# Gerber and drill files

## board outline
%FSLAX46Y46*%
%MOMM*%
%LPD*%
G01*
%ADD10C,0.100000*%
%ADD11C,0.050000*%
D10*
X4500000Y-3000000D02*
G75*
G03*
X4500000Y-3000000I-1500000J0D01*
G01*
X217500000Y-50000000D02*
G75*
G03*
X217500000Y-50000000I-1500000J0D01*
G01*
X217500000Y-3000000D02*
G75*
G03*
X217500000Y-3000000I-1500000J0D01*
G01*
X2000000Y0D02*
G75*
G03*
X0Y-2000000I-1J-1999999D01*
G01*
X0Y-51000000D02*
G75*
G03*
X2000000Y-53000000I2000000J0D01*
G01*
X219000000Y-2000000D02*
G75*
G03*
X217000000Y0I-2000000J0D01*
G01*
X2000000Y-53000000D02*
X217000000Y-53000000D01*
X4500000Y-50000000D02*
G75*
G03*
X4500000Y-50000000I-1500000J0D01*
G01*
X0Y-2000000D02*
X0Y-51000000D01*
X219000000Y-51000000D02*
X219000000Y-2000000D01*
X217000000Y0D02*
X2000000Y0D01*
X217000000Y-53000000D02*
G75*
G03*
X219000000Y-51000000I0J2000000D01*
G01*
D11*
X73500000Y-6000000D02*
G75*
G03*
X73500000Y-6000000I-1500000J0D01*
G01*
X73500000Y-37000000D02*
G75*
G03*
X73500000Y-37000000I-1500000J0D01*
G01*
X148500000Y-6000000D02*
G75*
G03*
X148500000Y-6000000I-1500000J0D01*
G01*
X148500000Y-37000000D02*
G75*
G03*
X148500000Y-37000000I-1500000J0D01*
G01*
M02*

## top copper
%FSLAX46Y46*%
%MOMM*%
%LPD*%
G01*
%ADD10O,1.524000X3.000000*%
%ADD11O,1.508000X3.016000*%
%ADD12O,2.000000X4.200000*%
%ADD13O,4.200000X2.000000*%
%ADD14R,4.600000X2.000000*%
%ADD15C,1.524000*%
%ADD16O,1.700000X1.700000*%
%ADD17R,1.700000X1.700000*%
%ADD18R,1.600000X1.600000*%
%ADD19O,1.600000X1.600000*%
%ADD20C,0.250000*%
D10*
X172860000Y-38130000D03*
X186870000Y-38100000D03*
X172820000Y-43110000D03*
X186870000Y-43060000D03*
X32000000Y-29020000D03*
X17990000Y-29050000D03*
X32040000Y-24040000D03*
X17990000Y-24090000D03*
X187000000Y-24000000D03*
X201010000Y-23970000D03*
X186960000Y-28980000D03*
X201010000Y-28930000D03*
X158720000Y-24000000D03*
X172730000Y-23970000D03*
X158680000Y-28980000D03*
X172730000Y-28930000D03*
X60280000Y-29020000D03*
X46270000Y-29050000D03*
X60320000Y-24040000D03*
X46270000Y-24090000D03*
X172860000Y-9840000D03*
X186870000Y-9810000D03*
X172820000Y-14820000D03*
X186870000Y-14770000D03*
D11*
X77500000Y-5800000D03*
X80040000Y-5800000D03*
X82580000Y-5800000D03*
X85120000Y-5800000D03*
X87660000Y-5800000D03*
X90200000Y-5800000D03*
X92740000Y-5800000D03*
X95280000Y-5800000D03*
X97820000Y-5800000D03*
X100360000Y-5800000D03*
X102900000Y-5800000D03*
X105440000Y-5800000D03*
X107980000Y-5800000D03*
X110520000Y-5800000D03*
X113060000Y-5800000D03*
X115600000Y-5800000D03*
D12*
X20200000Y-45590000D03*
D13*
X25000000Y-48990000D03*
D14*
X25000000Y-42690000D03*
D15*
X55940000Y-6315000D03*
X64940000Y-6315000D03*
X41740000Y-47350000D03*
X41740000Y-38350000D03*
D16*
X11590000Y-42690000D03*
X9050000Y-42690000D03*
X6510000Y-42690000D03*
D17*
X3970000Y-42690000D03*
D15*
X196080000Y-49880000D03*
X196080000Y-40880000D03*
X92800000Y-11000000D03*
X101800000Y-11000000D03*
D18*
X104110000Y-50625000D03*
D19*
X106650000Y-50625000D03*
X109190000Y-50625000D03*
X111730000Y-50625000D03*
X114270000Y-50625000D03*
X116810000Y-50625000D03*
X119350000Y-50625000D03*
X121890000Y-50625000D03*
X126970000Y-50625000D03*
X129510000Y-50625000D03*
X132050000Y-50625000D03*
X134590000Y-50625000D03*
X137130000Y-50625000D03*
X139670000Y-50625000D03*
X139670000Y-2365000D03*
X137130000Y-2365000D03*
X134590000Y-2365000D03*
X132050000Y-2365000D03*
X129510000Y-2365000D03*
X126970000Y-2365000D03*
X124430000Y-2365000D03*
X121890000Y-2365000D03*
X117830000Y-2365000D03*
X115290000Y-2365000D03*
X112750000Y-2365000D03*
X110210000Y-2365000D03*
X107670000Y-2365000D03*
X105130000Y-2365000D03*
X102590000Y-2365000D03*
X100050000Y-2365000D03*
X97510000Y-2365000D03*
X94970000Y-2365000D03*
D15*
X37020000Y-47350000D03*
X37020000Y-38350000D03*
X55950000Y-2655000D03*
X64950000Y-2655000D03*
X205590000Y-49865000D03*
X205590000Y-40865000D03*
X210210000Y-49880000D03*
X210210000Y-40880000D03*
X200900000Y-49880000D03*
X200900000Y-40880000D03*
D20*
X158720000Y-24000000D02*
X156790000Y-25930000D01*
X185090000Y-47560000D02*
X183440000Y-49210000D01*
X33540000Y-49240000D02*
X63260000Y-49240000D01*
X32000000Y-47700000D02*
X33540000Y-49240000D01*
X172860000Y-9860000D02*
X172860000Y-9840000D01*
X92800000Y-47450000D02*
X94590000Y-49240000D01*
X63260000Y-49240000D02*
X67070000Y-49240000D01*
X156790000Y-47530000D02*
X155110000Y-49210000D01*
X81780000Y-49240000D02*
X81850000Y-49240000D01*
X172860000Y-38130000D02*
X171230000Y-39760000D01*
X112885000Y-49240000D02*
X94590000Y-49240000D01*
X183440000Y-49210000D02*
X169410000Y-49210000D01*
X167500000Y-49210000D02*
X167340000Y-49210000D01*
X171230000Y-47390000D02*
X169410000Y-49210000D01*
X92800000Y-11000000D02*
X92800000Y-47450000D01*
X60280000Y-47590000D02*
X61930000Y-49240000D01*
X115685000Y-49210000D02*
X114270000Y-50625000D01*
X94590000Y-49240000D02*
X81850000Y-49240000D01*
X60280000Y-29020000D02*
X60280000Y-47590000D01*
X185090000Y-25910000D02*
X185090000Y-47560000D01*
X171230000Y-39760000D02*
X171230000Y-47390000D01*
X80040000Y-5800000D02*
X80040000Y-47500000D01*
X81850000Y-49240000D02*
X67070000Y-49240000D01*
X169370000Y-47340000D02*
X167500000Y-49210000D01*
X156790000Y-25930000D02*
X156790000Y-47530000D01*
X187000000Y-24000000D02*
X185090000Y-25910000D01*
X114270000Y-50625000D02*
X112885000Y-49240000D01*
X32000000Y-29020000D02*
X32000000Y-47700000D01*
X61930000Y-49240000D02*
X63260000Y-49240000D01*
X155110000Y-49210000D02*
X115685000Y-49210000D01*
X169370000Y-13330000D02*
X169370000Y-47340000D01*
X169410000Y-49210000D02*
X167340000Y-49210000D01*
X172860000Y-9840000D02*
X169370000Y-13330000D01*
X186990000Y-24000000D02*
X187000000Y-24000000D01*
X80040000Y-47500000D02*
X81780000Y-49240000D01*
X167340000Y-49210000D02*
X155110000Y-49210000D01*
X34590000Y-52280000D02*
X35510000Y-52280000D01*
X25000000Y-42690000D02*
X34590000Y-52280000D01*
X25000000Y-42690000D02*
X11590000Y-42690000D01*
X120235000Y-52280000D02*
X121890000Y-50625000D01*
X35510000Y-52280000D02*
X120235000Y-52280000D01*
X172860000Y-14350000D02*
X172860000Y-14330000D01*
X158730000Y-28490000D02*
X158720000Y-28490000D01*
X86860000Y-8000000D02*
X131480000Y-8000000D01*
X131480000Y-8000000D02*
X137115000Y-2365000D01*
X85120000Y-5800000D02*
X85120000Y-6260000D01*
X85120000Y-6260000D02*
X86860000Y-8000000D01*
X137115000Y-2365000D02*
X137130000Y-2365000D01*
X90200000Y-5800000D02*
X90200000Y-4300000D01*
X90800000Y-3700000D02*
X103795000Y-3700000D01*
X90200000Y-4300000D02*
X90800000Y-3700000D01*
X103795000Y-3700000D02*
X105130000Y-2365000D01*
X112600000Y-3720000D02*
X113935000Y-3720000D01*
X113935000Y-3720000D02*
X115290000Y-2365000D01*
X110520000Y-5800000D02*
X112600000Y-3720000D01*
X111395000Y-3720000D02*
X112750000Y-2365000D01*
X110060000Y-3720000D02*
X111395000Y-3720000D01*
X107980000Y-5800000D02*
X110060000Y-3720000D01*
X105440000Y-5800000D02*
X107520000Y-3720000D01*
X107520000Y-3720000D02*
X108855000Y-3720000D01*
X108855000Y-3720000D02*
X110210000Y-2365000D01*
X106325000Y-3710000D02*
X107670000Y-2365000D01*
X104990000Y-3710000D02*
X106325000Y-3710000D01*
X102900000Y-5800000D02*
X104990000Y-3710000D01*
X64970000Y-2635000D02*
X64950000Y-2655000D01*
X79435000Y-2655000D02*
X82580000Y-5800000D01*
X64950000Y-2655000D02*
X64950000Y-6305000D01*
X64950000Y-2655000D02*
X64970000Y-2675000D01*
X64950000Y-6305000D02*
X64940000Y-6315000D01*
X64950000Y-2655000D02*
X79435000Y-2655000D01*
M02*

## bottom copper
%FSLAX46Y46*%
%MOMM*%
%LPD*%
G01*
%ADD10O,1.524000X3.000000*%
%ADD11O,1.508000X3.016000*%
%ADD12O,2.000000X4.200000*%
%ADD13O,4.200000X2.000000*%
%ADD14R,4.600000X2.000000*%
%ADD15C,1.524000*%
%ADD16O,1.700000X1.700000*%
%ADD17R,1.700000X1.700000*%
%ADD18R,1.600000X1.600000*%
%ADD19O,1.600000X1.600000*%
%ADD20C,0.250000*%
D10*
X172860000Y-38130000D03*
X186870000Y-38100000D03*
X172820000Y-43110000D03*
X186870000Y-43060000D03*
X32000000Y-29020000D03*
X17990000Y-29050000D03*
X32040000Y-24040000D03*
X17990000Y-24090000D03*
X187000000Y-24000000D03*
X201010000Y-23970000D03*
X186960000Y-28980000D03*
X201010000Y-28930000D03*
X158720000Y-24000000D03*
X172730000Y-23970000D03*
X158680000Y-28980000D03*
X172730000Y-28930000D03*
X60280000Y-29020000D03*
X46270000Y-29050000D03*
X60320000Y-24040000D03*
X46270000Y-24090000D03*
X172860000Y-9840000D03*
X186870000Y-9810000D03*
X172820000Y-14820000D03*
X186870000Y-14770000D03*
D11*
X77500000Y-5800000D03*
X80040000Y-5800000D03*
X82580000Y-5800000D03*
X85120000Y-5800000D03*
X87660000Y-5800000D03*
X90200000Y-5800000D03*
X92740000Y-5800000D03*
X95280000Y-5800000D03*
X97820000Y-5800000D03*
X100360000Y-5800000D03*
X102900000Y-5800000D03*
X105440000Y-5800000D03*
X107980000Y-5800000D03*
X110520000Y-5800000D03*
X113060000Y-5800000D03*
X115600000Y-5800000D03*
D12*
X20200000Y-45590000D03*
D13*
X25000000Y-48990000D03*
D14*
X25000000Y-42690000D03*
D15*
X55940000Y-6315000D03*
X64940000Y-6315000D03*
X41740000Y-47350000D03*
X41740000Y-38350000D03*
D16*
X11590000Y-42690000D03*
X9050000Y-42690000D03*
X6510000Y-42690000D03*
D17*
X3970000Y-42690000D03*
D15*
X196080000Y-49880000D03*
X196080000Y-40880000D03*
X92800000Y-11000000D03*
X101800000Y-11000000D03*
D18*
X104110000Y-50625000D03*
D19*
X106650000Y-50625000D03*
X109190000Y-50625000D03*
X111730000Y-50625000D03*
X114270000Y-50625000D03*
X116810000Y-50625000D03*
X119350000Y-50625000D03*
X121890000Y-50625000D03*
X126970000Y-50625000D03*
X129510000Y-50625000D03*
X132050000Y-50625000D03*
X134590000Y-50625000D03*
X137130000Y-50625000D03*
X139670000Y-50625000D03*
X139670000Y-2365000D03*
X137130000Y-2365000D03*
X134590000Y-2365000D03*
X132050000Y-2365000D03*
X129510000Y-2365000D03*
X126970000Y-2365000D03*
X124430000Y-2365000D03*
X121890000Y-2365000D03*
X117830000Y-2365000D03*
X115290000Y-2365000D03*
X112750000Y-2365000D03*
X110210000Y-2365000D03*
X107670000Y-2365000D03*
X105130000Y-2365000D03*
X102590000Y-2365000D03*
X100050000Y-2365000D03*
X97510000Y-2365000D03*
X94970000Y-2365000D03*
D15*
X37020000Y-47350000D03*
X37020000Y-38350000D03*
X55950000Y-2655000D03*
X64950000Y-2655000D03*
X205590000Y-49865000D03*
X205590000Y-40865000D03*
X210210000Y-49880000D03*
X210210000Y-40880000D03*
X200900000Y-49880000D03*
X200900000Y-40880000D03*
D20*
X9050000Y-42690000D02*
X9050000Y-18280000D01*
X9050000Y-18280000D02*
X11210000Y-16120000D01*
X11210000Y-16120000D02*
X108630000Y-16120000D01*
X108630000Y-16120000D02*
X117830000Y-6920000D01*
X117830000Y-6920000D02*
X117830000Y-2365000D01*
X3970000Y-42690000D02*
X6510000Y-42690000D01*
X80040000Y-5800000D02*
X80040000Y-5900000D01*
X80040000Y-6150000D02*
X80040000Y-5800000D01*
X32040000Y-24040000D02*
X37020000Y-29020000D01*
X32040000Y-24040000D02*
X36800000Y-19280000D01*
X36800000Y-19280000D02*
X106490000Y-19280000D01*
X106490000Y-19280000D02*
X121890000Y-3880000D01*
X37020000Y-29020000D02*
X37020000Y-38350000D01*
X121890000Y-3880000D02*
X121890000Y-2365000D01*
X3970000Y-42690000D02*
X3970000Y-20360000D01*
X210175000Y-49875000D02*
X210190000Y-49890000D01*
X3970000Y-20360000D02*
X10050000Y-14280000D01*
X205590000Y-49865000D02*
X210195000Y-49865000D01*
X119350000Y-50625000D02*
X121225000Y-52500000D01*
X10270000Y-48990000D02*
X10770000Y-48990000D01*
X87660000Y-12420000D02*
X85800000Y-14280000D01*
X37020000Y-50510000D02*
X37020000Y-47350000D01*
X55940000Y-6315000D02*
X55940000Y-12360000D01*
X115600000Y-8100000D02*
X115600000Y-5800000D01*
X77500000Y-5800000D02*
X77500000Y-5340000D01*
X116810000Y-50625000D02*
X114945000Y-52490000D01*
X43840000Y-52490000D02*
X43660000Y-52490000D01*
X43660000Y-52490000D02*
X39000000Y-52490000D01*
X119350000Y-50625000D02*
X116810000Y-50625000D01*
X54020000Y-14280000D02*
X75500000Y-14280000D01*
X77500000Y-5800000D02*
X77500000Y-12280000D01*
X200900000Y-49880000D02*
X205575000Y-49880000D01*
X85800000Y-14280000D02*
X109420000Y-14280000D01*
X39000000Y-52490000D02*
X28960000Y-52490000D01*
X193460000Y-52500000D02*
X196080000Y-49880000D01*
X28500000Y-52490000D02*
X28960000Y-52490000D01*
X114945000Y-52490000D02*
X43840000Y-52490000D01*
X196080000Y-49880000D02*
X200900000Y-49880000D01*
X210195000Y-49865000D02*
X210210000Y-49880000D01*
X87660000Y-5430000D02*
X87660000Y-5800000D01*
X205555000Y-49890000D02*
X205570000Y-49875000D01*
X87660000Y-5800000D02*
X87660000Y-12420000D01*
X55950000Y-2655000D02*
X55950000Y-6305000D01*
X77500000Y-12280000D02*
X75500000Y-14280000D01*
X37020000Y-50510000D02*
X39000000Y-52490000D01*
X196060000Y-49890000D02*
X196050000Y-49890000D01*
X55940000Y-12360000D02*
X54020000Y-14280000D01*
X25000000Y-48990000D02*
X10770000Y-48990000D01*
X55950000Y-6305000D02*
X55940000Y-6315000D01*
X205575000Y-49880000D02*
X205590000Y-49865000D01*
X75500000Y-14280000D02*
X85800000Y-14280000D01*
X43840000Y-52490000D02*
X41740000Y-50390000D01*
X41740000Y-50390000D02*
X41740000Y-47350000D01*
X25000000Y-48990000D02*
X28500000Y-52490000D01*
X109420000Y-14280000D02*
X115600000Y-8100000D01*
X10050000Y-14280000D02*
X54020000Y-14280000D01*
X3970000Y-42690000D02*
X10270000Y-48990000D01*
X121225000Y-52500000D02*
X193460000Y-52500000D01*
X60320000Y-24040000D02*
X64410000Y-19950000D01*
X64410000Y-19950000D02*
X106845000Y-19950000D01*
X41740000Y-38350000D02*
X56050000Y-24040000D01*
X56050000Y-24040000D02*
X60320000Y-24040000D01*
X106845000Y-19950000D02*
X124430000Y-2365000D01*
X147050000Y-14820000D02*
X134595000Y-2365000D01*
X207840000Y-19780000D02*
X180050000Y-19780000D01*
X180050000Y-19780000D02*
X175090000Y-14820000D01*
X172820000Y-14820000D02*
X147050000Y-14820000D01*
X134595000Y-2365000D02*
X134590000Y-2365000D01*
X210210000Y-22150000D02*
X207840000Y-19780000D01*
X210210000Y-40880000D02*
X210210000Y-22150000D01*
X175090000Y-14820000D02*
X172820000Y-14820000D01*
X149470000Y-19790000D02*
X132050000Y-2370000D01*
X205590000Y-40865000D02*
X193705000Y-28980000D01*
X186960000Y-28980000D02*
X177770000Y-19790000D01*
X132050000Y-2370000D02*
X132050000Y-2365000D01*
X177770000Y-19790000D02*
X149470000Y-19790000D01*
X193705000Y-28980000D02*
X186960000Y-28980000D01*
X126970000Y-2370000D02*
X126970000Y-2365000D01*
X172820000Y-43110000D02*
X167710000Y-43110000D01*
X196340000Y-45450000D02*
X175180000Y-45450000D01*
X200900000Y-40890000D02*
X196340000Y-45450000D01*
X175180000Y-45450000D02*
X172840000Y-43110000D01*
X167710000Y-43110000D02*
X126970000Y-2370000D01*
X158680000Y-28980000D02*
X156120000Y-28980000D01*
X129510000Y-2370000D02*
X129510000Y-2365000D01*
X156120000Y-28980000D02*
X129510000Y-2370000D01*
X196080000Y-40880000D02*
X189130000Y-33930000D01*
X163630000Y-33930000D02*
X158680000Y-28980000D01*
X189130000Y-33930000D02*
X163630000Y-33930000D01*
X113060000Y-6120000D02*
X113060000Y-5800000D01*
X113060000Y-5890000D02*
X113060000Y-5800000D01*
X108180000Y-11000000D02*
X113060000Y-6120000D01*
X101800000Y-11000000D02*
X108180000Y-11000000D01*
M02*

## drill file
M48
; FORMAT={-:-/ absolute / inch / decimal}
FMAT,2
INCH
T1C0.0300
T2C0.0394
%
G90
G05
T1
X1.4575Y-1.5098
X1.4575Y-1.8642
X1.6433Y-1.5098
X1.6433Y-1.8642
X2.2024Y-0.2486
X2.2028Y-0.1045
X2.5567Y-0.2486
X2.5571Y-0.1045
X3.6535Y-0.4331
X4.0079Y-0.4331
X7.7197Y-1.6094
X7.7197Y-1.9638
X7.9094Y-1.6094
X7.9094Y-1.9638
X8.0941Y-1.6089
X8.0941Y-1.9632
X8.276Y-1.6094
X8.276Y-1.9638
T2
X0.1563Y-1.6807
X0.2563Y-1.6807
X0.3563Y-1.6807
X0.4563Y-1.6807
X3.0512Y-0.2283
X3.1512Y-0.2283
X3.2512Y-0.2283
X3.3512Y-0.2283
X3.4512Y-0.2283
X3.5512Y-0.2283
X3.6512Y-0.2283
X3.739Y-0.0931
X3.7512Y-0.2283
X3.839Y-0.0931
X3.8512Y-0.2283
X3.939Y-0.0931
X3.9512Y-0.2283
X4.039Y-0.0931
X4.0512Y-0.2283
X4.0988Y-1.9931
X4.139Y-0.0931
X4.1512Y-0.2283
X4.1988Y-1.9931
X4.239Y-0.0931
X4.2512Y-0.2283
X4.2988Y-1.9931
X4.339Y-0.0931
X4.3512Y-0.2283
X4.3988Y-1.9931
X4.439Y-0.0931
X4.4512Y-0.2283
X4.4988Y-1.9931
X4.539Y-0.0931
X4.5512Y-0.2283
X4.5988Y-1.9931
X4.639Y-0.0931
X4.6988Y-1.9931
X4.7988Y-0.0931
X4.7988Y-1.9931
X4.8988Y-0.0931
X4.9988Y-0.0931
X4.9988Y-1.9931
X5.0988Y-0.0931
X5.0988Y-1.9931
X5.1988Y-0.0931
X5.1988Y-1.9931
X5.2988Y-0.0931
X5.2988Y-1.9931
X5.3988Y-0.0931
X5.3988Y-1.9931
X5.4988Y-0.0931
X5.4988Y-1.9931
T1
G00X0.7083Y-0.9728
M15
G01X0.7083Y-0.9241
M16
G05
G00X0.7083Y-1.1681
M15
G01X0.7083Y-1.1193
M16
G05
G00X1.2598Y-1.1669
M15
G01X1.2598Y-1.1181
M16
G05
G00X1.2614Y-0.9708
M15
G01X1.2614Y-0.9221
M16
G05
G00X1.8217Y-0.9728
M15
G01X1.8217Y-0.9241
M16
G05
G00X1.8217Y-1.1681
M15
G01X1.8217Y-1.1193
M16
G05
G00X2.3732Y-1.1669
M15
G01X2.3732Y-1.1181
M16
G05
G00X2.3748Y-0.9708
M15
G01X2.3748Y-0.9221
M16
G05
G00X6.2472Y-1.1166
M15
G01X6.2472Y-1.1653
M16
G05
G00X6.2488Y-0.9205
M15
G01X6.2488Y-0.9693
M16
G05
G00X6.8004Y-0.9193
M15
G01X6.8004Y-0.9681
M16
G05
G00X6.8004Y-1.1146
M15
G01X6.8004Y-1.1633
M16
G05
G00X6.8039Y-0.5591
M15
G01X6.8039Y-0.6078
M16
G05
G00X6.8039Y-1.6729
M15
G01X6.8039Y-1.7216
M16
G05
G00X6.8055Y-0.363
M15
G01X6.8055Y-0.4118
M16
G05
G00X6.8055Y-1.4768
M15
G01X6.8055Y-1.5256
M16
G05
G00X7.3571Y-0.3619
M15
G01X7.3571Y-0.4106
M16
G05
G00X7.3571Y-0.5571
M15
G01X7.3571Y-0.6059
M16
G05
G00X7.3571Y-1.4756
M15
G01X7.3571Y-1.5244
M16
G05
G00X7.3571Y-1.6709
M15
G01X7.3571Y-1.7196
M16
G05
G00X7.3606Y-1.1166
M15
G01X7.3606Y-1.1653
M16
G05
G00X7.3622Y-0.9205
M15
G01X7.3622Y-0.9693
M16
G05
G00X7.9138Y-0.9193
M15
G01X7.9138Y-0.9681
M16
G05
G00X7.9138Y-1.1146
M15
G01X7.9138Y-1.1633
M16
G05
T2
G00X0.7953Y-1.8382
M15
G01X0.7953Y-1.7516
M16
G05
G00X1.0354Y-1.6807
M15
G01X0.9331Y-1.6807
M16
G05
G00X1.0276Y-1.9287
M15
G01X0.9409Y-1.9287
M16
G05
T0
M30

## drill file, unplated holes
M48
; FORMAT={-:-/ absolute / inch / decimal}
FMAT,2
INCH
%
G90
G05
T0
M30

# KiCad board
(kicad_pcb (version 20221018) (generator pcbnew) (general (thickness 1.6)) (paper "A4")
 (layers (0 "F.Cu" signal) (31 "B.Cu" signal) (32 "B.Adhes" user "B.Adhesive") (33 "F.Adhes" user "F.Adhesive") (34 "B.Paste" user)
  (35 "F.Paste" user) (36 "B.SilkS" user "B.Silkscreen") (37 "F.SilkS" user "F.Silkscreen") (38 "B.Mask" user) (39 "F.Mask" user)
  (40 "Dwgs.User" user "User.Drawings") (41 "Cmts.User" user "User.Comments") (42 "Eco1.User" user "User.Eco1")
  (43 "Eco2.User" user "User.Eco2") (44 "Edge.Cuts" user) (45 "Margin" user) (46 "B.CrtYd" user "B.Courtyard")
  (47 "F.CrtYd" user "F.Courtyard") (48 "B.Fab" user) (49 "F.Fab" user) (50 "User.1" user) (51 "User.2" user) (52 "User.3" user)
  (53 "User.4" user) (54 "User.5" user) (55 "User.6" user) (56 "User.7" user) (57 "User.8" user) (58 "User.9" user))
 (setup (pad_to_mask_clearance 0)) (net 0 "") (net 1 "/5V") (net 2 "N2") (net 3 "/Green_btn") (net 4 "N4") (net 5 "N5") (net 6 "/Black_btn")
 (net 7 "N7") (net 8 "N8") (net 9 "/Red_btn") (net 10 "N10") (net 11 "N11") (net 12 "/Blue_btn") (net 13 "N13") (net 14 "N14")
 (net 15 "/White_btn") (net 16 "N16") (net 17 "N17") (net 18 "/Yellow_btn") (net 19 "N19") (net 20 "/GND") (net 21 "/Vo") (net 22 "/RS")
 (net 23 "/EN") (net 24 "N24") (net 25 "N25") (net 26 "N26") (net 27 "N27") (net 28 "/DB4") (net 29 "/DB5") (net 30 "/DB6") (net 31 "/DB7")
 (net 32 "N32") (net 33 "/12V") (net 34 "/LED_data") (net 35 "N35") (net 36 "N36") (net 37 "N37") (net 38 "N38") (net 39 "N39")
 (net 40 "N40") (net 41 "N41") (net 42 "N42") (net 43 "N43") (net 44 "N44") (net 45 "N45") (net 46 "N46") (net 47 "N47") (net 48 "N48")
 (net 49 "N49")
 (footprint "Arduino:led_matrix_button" (layer "F.Cu") (at 179.86 40.64)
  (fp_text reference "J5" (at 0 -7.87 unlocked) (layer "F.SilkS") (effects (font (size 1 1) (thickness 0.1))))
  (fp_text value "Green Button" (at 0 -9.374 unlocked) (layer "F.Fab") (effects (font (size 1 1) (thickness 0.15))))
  (pad "1" thru_hole oval (at -7 -2.51) (size 1.524 3) (drill oval 0.762 2) (layers "*.Cu" "*.Mask") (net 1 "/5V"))
  (pad "2" thru_hole oval (at 7.01 -2.54) (size 1.524 3) (drill oval 0.762 2) (layers "*.Cu" "*.Mask") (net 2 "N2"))
  (pad "3" thru_hole oval (at -7.04 2.47) (size 1.524 3) (drill oval 0.762 2) (layers "*.Cu" "*.Mask") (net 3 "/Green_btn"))
  (pad "4" thru_hole oval (at 7.01 2.42) (size 1.524 3) (drill oval 0.762 2) (layers "*.Cu" "*.Mask") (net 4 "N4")))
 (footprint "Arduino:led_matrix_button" (layer "F.Cu") (at 25 26.51 180)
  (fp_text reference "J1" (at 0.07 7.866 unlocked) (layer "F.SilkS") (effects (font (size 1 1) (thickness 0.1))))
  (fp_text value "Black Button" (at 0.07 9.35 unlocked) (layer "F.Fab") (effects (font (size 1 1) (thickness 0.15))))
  (pad "1" thru_hole oval (at -7 -2.51 180) (size 1.524 3) (drill oval 0.762 2) (layers "*.Cu" "*.Mask") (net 1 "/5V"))
  (pad "2" thru_hole oval (at 7.01 -2.54 180) (size 1.524 3) (drill oval 0.762 2) (layers "*.Cu" "*.Mask") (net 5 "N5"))
  (pad "3" thru_hole oval (at -7.04 2.47 180) (size 1.524 3) (drill oval 0.762 2) (layers "*.Cu" "*.Mask") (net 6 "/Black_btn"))
  (pad "4" thru_hole oval (at 7.01 2.42 180) (size 1.524 3) (drill oval 0.762 2) (layers "*.Cu" "*.Mask") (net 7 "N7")))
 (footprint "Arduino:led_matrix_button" (layer "F.Cu") (at 194 26.51)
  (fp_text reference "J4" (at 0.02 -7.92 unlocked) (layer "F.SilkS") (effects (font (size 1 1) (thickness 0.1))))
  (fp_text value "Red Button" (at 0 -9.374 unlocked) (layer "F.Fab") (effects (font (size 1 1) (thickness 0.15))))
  (pad "1" thru_hole oval (at -7 -2.51) (size 1.524 3) (drill oval 0.762 2) (layers "*.Cu" "*.Mask") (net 1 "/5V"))
  (pad "2" thru_hole oval (at 7.01 -2.54) (size 1.524 3) (drill oval 0.762 2) (layers "*.Cu" "*.Mask") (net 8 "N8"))
  (pad "3" thru_hole oval (at -7.04 2.47) (size 1.524 3) (drill oval 0.762 2) (layers "*.Cu" "*.Mask") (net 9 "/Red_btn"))
  (pad "4" thru_hole oval (at 7.01 2.42) (size 1.524 3) (drill oval 0.762 2) (layers "*.Cu" "*.Mask") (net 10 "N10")))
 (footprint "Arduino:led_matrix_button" (layer "F.Cu") (at 165.72 26.51)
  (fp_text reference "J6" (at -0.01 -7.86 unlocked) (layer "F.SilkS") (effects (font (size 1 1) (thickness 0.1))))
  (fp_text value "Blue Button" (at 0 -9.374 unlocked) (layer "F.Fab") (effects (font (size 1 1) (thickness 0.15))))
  (pad "1" thru_hole oval (at -7 -2.51) (size 1.524 3) (drill oval 0.762 2) (layers "*.Cu" "*.Mask") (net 1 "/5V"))
  (pad "2" thru_hole oval (at 7.01 -2.54) (size 1.524 3) (drill oval 0.762 2) (layers "*.Cu" "*.Mask") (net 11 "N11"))
  (pad "3" thru_hole oval (at -7.04 2.47) (size 1.524 3) (drill oval 0.762 2) (layers "*.Cu" "*.Mask") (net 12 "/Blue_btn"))
  (pad "4" thru_hole oval (at 7.01 2.42) (size 1.524 3) (drill oval 0.762 2) (layers "*.Cu" "*.Mask") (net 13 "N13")))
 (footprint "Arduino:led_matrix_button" (layer "F.Cu") (at 53.28 26.51 180)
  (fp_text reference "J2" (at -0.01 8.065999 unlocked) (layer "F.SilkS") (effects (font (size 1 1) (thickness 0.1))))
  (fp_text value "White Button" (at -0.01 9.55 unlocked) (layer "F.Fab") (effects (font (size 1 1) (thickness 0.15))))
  (pad "1" thru_hole oval (at -7 -2.51 180) (size 1.524 3) (drill oval 0.762 2) (layers "*.Cu" "*.Mask") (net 1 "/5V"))
  (pad "2" thru_hole oval (at 7.01 -2.54 180) (size 1.524 3) (drill oval 0.762 2) (layers "*.Cu" "*.Mask") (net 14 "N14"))
  (pad "3" thru_hole oval (at -7.04 2.47 180) (size 1.524 3) (drill oval 0.762 2) (layers "*.Cu" "*.Mask") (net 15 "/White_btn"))
  (pad "4" thru_hole oval (at 7.01 2.42 180) (size 1.524 3) (drill oval 0.762 2) (layers "*.Cu" "*.Mask") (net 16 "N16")))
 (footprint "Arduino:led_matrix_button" (layer "F.Cu") (at 179.86 12.35)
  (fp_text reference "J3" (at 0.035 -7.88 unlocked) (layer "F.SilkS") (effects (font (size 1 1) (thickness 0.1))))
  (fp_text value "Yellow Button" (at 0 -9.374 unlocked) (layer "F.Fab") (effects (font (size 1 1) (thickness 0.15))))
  (pad "1" thru_hole oval (at -7 -2.51) (size 1.524 3) (drill oval 0.762 2) (layers "*.Cu" "*.Mask") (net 1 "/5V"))
  (pad "2" thru_hole oval (at 7.01 -2.54) (size 1.524 3) (drill oval 0.762 2) (layers "*.Cu" "*.Mask") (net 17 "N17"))
  (pad "3" thru_hole oval (at -7.04 2.47) (size 1.524 3) (drill oval 0.762 2) (layers "*.Cu" "*.Mask") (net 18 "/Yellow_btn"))
  (pad "4" thru_hole oval (at 7.01 2.42) (size 1.524 3) (drill oval 0.762 2) (layers "*.Cu" "*.Mask") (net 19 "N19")))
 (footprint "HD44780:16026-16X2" (layer "F.Cu") (at 69.5 3.5)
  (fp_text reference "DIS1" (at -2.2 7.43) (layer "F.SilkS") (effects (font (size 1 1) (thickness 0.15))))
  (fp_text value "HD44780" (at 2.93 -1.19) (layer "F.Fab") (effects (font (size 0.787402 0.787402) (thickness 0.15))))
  (fp_circle (center 2.5 2.5) (end 4 2.5) (stroke (width 0.05) (type default)) (fill none) (layer "Edge.Cuts"))
  (fp_circle (center 2.5 33.5) (end 4 33.5) (stroke (width 0.05) (type default)) (fill none) (layer "Edge.Cuts"))
  (fp_circle (center 77.5 2.5) (end 79 2.5) (stroke (width 0.05) (type default)) (fill none) (layer "Edge.Cuts"))
  (fp_circle (center 77.5 33.5) (end 79 33.5) (stroke (width 0.05) (type default)) (fill none) (layer "Edge.Cuts"))
  (pad "P$1" thru_hole oval (at 8 2.3) (size 1.508 3.016) (drill 1) (layers "*.Cu" "*.Mask") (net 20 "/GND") (solder_mask_margin 0.102))
  (pad "P$2" thru_hole oval (at 10.54 2.3) (size 1.508 3.016) (drill 1) (layers "*.Cu" "*.Mask") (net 1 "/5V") (solder_mask_margin 0.102))
  (pad "P$3" thru_hole oval (at 13.08 2.3) (size 1.508 3.016) (drill 1) (layers "*.Cu" "*.Mask") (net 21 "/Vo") (solder_mask_margin 0.102))
  (pad "P$4" thru_hole oval (at 15.62 2.3) (size 1.508 3.016) (drill 1) (layers "*.Cu" "*.Mask") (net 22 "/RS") (solder_mask_margin 0.102))
  (pad "P$5" thru_hole oval (at 18.16 2.3) (size 1.508 3.016) (drill 1) (layers "*.Cu" "*.Mask") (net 20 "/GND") (solder_mask_margin 0.102))
  (pad "P$6" thru_hole oval (at 20.7 2.3) (size 1.508 3.016) (drill 1) (layers "*.Cu" "*.Mask") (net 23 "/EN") (solder_mask_margin 0.102))
  (pad "P$7" thru_hole oval (at 23.24 2.3) (size 1.508 3.016) (drill 1) (layers "*.Cu" "*.Mask") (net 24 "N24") (solder_mask_margin 0.102))
  (pad "P$8" thru_hole oval (at 25.78 2.3) (size 1.508 3.016) (drill 1) (layers "*.Cu" "*.Mask") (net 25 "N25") (solder_mask_margin 0.102))
  (pad "P$9" thru_hole oval (at 28.32 2.3) (size 1.508 3.016) (drill 1) (layers "*.Cu" "*.Mask") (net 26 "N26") (solder_mask_margin 0.102))
  (pad "P$10" thru_hole oval (at 30.86 2.3) (size 1.508 3.016) (drill 1) (layers "*.Cu" "*.Mask") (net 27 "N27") (solder_mask_margin 0.102))
  (pad "P$11" thru_hole oval (at 33.4 2.3) (size 1.508 3.016) (drill 1) (layers "*.Cu" "*.Mask") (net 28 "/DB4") (solder_mask_margin 0.102))
  (pad "P$12" thru_hole oval (at 35.94 2.3) (size 1.508 3.016) (drill 1) (layers "*.Cu" "*.Mask") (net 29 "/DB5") (solder_mask_margin 0.102))
  (pad "P$13" thru_hole oval (at 38.48 2.3) (size 1.508 3.016) (drill 1) (layers "*.Cu" "*.Mask") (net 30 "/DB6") (solder_mask_margin 0.102))
  (pad "P$14" thru_hole oval (at 41.02 2.3) (size 1.508 3.016) (drill 1) (layers "*.Cu" "*.Mask") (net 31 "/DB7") (solder_mask_margin 0.102))
  (pad "P$15" thru_hole oval (at 43.56 2.3) (size 1.508 3.016) (drill 1) (layers "*.Cu" "*.Mask") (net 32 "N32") (solder_mask_margin 0.102))
  (pad "P$16" thru_hole oval (at 46.1 2.3) (size 1.508 3.016) (drill 1) (layers "*.Cu" "*.Mask") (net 20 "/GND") (solder_mask_margin 0.102)))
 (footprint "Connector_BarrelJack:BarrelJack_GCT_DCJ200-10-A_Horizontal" (layer "B.Cu") (at 25 42.69 180)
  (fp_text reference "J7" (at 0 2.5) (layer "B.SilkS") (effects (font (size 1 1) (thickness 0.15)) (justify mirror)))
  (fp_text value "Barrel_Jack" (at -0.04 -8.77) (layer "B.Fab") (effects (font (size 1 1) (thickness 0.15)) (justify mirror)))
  (pad "1" thru_hole rect (at 0 0 180) (size 4.6 2) (drill oval 3.6 1) (layers "*.Cu" "*.Mask") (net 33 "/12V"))
  (pad "2" thru_hole oval (at 0 -6.3 180) (size 4.2 2) (drill oval 3.2 1) (layers "*.Cu" "*.Mask") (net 20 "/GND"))
  (pad "3" thru_hole oval (at 4.8 -2.9 180) (size 2 4.2) (drill oval 1 3.2) (layers "*.Cu" "*.Mask")))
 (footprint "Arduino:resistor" (layer "B.Cu") (at 60.44 6.315 -90)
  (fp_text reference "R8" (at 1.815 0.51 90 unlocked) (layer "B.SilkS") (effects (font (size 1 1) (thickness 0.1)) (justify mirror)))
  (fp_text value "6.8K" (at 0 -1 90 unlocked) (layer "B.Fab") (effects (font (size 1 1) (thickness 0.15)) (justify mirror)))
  (pad "1" thru_hole circle (at 0 4.5 270) (size 1.524 1.524) (drill 0.762) (layers "*.Cu" "*.Mask") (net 20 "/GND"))
  (pad "2" thru_hole circle (at 0 -4.5 270) (size 1.524 1.524) (drill 0.762) (layers "*.Cu" "*.Mask") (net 21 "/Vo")))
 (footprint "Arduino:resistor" (layer "B.Cu") (at 41.74 42.85)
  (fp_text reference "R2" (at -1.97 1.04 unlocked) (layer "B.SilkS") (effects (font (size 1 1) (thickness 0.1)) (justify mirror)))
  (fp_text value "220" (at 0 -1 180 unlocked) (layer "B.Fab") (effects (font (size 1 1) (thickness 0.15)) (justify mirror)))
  (pad "1" thru_hole circle (at 0 4.5) (size 1.524 1.524) (drill 0.762) (layers "*.Cu" "*.Mask") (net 20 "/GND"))
  (pad "2" thru_hole circle (at 0 -4.5) (size 1.524 1.524) (drill 0.762) (layers "*.Cu" "*.Mask") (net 15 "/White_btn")))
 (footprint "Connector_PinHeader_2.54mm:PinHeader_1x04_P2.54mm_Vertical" (layer "B.Cu") (at 3.97 42.69 -90)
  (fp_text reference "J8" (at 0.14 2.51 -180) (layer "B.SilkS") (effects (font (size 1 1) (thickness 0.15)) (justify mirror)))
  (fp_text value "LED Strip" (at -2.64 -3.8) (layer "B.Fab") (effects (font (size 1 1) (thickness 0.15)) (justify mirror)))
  (pad "1" thru_hole rect (at 0 0 270) (size 1.7 1.7) (drill 1) (layers "*.Cu" "*.Mask") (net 20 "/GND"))
  (pad "2" thru_hole oval (at 0 -2.54 270) (size 1.7 1.7) (drill 1) (layers "*.Cu" "*.Mask") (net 20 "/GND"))
  (pad "3" thru_hole oval (at 0 -5.08 270) (size 1.7 1.7) (drill 1) (layers "*.Cu" "*.Mask") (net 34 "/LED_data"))
  (pad "4" thru_hole oval (at 0 -7.62 270) (size 1.7 1.7) (drill 1) (layers "*.Cu" "*.Mask") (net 33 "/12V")))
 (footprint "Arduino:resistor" (layer "B.Cu") (at 196.08 45.38)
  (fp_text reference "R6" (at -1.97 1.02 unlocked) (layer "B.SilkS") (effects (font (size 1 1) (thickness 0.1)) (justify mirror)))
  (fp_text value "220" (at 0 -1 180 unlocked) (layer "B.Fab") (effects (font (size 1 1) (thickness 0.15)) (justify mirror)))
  (pad "1" thru_hole circle (at 0 4.5) (size 1.524 1.524) (drill 0.762) (layers "*.Cu" "*.Mask") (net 20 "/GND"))
  (pad "2" thru_hole circle (at 0 -4.5) (size 1.524 1.524) (drill 0.762) (layers "*.Cu" "*.Mask") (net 12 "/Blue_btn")))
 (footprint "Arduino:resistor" (layer "B.Cu") (at 97.3 11 -90)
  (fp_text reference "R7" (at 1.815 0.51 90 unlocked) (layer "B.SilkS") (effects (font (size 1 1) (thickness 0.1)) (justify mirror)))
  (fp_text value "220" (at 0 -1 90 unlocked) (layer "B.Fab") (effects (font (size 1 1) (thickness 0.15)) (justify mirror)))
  (pad "1" thru_hole circle (at 0 4.5 270) (size 1.524 1.524) (drill 0.762) (layers "*.Cu" "*.Mask") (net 1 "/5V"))
  (pad "2" thru_hole circle (at 0 -4.5 270) (size 1.524 1.524) (drill 0.762) (layers "*.Cu" "*.Mask") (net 32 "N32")))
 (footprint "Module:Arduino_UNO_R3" (layer "B.Cu") (at 104.11 50.625)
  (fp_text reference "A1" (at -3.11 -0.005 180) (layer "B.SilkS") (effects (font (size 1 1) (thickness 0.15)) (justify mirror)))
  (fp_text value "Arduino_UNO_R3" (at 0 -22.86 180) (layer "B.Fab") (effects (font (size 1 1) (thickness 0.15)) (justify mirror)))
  (pad "1" thru_hole rect (at 0 0 270) (size 1.6 1.6) (drill 1) (layers "*.Cu" "*.Mask") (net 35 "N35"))
  (pad "2" thru_hole oval (at 2.54 0 270) (size 1.6 1.6) (drill 1) (layers "*.Cu" "*.Mask") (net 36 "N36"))
  (pad "3" thru_hole oval (at 5.08 0 270) (size 1.6 1.6) (drill 1) (layers "*.Cu" "*.Mask") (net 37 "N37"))
  (pad "4" thru_hole oval (at 7.62 0 270) (size 1.6 1.6) (drill 1) (layers "*.Cu" "*.Mask") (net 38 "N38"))
  (pad "5" thru_hole oval (at 10.16 0 270) (size 1.6 1.6) (drill 1) (layers "*.Cu" "*.Mask") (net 1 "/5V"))
  (pad "6" thru_hole oval (at 12.7 0 270) (size 1.6 1.6) (drill 1) (layers "*.Cu" "*.Mask") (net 20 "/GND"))
  (pad "7" thru_hole oval (at 15.24 0 270) (size 1.6 1.6) (drill 1) (layers "*.Cu" "*.Mask") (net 20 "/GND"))
  (pad "8" thru_hole oval (at 17.78 0 270) (size 1.6 1.6) (drill 1) (layers "*.Cu" "*.Mask") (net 33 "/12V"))
  (pad "9" thru_hole oval (at 22.86 0 270) (size 1.6 1.6) (drill 1) (layers "*.Cu" "*.Mask") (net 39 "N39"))
  (pad "10" thru_hole oval (at 25.4 0 270) (size 1.6 1.6) (drill 1) (layers "*.Cu" "*.Mask") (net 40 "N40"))
  (pad "11" thru_hole oval (at 27.94 0 270) (size 1.6 1.6) (drill 1) (layers "*.Cu" "*.Mask") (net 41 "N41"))
  (pad "12" thru_hole oval (at 30.48 0 270) (size 1.6 1.6) (drill 1) (layers "*.Cu" "*.Mask") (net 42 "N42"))
  (pad "13" thru_hole oval (at 33.02 0 270) (size 1.6 1.6) (drill 1) (layers "*.Cu" "*.Mask") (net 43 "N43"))
  (pad "14" thru_hole oval (at 35.56 0 270) (size 1.6 1.6) (drill 1) (layers "*.Cu" "*.Mask") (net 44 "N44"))
  (pad "15" thru_hole oval (at 35.56 -48.26 270) (size 1.6 1.6) (drill 1) (layers "*.Cu" "*.Mask") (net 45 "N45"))
  (pad "16" thru_hole oval (at 33.02 -48.26 270) (size 1.6 1.6) (drill 1) (layers "*.Cu" "*.Mask") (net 22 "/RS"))
  (pad "17" thru_hole oval (at 30.48 -48.26 270) (size 1.6 1.6) (drill 1) (layers "*.Cu" "*.Mask") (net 18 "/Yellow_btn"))
  (pad "18" thru_hole oval (at 27.94 -48.26 270) (size 1.6 1.6) (drill 1) (layers "*.Cu" "*.Mask") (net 9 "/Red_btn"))
  (pad "19" thru_hole oval (at 25.4 -48.26 270) (size 1.6 1.6) (drill 1) (layers "*.Cu" "*.Mask") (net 12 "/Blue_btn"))
  (pad "20" thru_hole oval (at 22.86 -48.26 270) (size 1.6 1.6) (drill 1) (layers "*.Cu" "*.Mask") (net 3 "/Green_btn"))
  (pad "21" thru_hole oval (at 20.32 -48.26 270) (size 1.6 1.6) (drill 1) (layers "*.Cu" "*.Mask") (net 15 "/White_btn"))
  (pad "22" thru_hole oval (at 17.78 -48.26 270) (size 1.6 1.6) (drill 1) (layers "*.Cu" "*.Mask") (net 6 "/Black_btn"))
  (pad "23" thru_hole oval (at 13.72 -48.26 270) (size 1.6 1.6) (drill 1) (layers "*.Cu" "*.Mask") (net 34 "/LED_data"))
  (pad "24" thru_hole oval (at 11.18 -48.26 270) (size 1.6 1.6) (drill 1) (layers "*.Cu" "*.Mask") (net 31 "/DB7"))
  (pad "25" thru_hole oval (at 8.64 -48.26 270) (size 1.6 1.6) (drill 1) (layers "*.Cu" "*.Mask") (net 30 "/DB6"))
  (pad "26" thru_hole oval (at 6.1 -48.26 270) (size 1.6 1.6) (drill 1) (layers "*.Cu" "*.Mask") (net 29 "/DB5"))
  (pad "27" thru_hole oval (at 3.56 -48.26 270) (size 1.6 1.6) (drill 1) (layers "*.Cu" "*.Mask") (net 28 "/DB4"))
  (pad "28" thru_hole oval (at 1.02 -48.26 270) (size 1.6 1.6) (drill 1) (layers "*.Cu" "*.Mask") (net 23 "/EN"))
  (pad "29" thru_hole oval (at -1.52 -48.26 270) (size 1.6 1.6) (drill 1) (layers "*.Cu" "*.Mask") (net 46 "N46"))
  (pad "30" thru_hole oval (at -4.06 -48.26 270) (size 1.6 1.6) (drill 1) (layers "*.Cu" "*.Mask") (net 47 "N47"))
  (pad "31" thru_hole oval (at -6.6 -48.26 270) (size 1.6 1.6) (drill 1) (layers "*.Cu" "*.Mask") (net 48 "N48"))
  (pad "32" thru_hole oval (at -9.14 -48.26 270) (size 1.6 1.6) (drill 1) (layers "*.Cu" "*.Mask") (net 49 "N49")))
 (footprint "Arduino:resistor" (layer "B.Cu") (at 37.02 42.85)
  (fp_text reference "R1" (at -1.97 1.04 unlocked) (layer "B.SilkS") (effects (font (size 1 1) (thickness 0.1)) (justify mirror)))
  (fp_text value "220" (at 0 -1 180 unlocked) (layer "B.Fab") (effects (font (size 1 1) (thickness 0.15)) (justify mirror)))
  (pad "1" thru_hole circle (at 0 4.5) (size 1.524 1.524) (drill 0.762) (layers "*.Cu" "*.Mask") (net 20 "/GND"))
  (pad "2" thru_hole circle (at 0 -4.5) (size 1.524 1.524) (drill 0.762) (layers "*.Cu" "*.Mask") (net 6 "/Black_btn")))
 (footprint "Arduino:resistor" (layer "B.Cu") (at 60.45 2.655 -90)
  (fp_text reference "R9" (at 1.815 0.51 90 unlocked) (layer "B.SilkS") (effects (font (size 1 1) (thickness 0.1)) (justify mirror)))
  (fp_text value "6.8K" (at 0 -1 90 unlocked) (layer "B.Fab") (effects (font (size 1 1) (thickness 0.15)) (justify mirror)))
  (pad "1" thru_hole circle (at 0 4.5 270) (size 1.524 1.524) (drill 0.762) (layers "*.Cu" "*.Mask") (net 20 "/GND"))
  (pad "2" thru_hole circle (at 0 -4.5 270) (size 1.524 1.524) (drill 0.762) (layers "*.Cu" "*.Mask") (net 21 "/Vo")))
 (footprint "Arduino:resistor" (layer "B.Cu") (at 205.59 45.365)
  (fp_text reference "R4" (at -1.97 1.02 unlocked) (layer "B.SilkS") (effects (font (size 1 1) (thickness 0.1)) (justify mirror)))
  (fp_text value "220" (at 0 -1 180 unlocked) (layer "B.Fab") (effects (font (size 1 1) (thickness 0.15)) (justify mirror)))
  (pad "1" thru_hole circle (at 0 4.5) (size 1.524 1.524) (drill 0.762) (layers "*.Cu" "*.Mask") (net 20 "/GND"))
  (pad "2" thru_hole circle (at 0 -4.5) (size 1.524 1.524) (drill 0.762) (layers "*.Cu" "*.Mask") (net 9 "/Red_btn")))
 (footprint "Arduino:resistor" (layer "B.Cu") (at 210.21 45.38)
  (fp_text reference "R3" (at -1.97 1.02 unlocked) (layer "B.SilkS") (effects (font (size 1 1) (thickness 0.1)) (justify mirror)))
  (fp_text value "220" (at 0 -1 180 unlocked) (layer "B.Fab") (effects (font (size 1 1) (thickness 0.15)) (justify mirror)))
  (pad "1" thru_hole circle (at 0 4.5) (size 1.524 1.524) (drill 0.762) (layers "*.Cu" "*.Mask") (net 20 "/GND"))
  (pad "2" thru_hole circle (at 0 -4.5) (size 1.524 1.524) (drill 0.762) (layers "*.Cu" "*.Mask") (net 18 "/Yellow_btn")))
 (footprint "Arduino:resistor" (layer "B.Cu") (at 200.9 45.38)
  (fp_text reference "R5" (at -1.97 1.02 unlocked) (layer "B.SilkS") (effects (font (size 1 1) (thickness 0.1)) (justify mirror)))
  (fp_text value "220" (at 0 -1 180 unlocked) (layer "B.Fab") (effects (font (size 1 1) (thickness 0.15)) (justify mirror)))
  (pad "1" thru_hole circle (at 0 4.5) (size 1.524 1.524) (drill 0.762) (layers "*.Cu" "*.Mask") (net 20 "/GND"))
  (pad "2" thru_hole circle (at 0 -4.5) (size 1.524 1.524) (drill 0.762) (layers "*.Cu" "*.Mask") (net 3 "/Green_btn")))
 (gr_circle (center 3 3) (end 4.5 3) (stroke (width 0.1) (type default)) (fill none) (layer "Edge.Cuts"))
 (gr_circle (center 216 50) (end 217.5 50) (stroke (width 0.1) (type default)) (fill none) (layer "Edge.Cuts"))
 (gr_circle (center 216 3) (end 217.5 3) (stroke (width 0.1) (type default)) (fill none) (layer "Edge.Cuts"))
 (gr_arc (start 0 2) (mid 0.585786 0.585786) (end 2 0) (stroke (width 0.1) (type default)) (layer "Edge.Cuts"))
 (gr_arc (start 2 53) (mid 0.585786 52.414214) (end 0 51) (stroke (width 0.1) (type default)) (layer "Edge.Cuts"))
 (gr_arc (start 217 0) (mid 218.414214 0.585786) (end 219 2) (stroke (width 0.1) (type default)) (layer "Edge.Cuts"))
 (gr_line (start 2 53) (end 217 53) (stroke (width 0.1) (type default)) (layer "Edge.Cuts"))
 (gr_circle (center 3 50) (end 4.5 50) (stroke (width 0.1) (type default)) (fill none) (layer "Edge.Cuts"))
 (gr_line (start 0 2) (end 0 51) (stroke (width 0.1) (type default)) (layer "Edge.Cuts"))
 (gr_line (start 219 51) (end 219 2) (stroke (width 0.1) (type default)) (layer "Edge.Cuts"))
 (gr_line (start 217 0) (end 2 0) (stroke (width 0.1) (type default)) (layer "Edge.Cuts"))
 (gr_arc (start 219 51) (mid 218.414214 52.414214) (end 217 53) (stroke (width 0.1) (type default)) (layer "Edge.Cuts"))
 (segment (start 158.72 24) (end 156.79 25.93) (width 0.25) (layer "F.Cu") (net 1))
 (segment (start 185.09 47.56) (end 183.44 49.21) (width 0.25) (layer "F.Cu") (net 1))
 (segment (start 33.54 49.24) (end 63.26 49.24) (width 0.25) (layer "F.Cu") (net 1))
 (segment (start 32 47.7) (end 33.54 49.24) (width 0.25) (layer "F.Cu") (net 1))
 (segment (start 172.86 9.86) (end 172.86 9.84) (width 0.25) (layer "F.Cu") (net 1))
 (segment (start 92.8 47.45) (end 94.59 49.24) (width 0.25) (layer "F.Cu") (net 1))
 (segment (start 63.26 49.24) (end 67.07 49.24) (width 0.25) (layer "F.Cu") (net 1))
 (segment (start 156.79 47.53) (end 155.11 49.21) (width 0.25) (layer "F.Cu") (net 1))
 (segment (start 81.78 49.24) (end 81.85 49.24) (width 0.25) (layer "F.Cu") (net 1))
 (segment (start 172.86 38.13) (end 171.23 39.76) (width 0.25) (layer "F.Cu") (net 1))
 (segment (start 112.885 49.24) (end 94.59 49.24) (width 0.25) (layer "F.Cu") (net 1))
 (segment (start 183.44 49.21) (end 169.41 49.21) (width 0.25) (layer "F.Cu") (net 1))
 (segment (start 167.5 49.21) (end 167.34 49.21) (width 0.25) (layer "F.Cu") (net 1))
 (segment (start 171.23 47.39) (end 169.41 49.21) (width 0.25) (layer "F.Cu") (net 1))
 (segment (start 92.8 11) (end 92.8 47.45) (width 0.25) (layer "F.Cu") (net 1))
 (segment (start 60.28 47.59) (end 61.93 49.24) (width 0.25) (layer "F.Cu") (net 1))
 (segment (start 115.685 49.21) (end 114.27 50.625) (width 0.25) (layer "F.Cu") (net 1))
 (segment (start 94.59 49.24) (end 81.85 49.24) (width 0.25) (layer "F.Cu") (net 1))
 (segment (start 60.28 29.02) (end 60.28 47.59) (width 0.25) (layer "F.Cu") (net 1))
 (segment (start 185.09 25.91) (end 185.09 47.56) (width 0.25) (layer "F.Cu") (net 1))
 (segment (start 171.23 39.76) (end 171.23 47.39) (width 0.25) (layer "F.Cu") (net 1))
 (segment (start 80.04 5.8) (end 80.04 47.5) (width 0.25) (layer "F.Cu") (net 1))
 (segment (start 81.85 49.24) (end 67.07 49.24) (width 0.25) (layer "F.Cu") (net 1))
 (segment (start 169.37 47.34) (end 167.5 49.21) (width 0.25) (layer "F.Cu") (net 1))
 (segment (start 156.79 25.93) (end 156.79 47.53) (width 0.25) (layer "F.Cu") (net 1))
 (segment (start 187 24) (end 185.09 25.91) (width 0.25) (layer "F.Cu") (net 1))
 (segment (start 114.27 50.625) (end 112.885 49.24) (width 0.25) (layer "F.Cu") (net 1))
 (segment (start 32 29.02) (end 32 47.7) (width 0.25) (layer "F.Cu") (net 1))
 (segment (start 61.93 49.24) (end 63.26 49.24) (width 0.25) (layer "F.Cu") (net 1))
 (segment (start 155.11 49.21) (end 115.685 49.21) (width 0.25) (layer "F.Cu") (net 1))
 (segment (start 169.37 13.33) (end 169.37 47.34) (width 0.25) (layer "F.Cu") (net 1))
 (segment (start 169.41 49.21) (end 167.34 49.21) (width 0.25) (layer "F.Cu") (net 1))
 (segment (start 172.86 9.84) (end 169.37 13.33) (width 0.25) (layer "F.Cu") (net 1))
 (segment (start 186.99 24) (end 187 24) (width 0.25) (layer "F.Cu") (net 1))
 (segment (start 80.04 47.5) (end 81.78 49.24) (width 0.25) (layer "F.Cu") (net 1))
 (segment (start 167.34 49.21) (end 155.11 49.21) (width 0.25) (layer "F.Cu") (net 1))
 (segment (start 80.04 5.8) (end 80.04 5.9) (width 0.25) (layer "B.Cu") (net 1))
 (segment (start 80.04 6.15) (end 80.04 5.8) (width 0.25) (layer "B.Cu") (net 1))
 (segment (start 32.04 24.04) (end 37.02 29.02) (width 0.25) (layer "B.Cu") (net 6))
 (segment (start 32.04 24.04) (end 36.8 19.28) (width 0.25) (layer "B.Cu") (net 6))
 (segment (start 36.8 19.28) (end 106.49 19.28) (width 0.25) (layer "B.Cu") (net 6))
 (segment (start 106.49 19.28) (end 121.89 3.88) (width 0.25) (layer "B.Cu") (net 6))
 (segment (start 37.02 29.02) (end 37.02 38.35) (width 0.25) (layer "B.Cu") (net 6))
 (segment (start 121.89 3.88) (end 121.89 2.365) (width 0.25) (layer "B.Cu") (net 6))
 (segment (start 34.59 52.28) (end 35.51 52.28) (width 0.25) (layer "F.Cu") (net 33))
 (segment (start 25 42.69) (end 34.59 52.28) (width 0.25) (layer "F.Cu") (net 33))
 (segment (start 25 42.69) (end 11.59 42.69) (width 0.25) (layer "F.Cu") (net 33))
 (segment (start 120.235 52.28) (end 121.89 50.625) (width 0.25) (layer "F.Cu") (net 33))
 (segment (start 35.51 52.28) (end 120.235 52.28) (width 0.25) (layer "F.Cu") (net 33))
 (segment (start 3.97 42.69) (end 3.97 20.36) (width 0.25) (layer "B.Cu") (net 20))
 (segment (start 210.175 49.875) (end 210.19 49.89) (width 0.25) (layer "B.Cu") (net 20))
 (segment (start 3.97 20.36) (end 10.05 14.28) (width 0.25) (layer "B.Cu") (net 20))
 (segment (start 205.59 49.865) (end 210.195 49.865) (width 0.25) (layer "B.Cu") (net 20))
 (segment (start 119.35 50.625) (end 121.225 52.5) (width 0.25) (layer "B.Cu") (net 20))
 (segment (start 10.27 48.99) (end 10.77 48.99) (width 0.25) (layer "B.Cu") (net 20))
 (segment (start 87.66 12.42) (end 85.8 14.28) (width 0.25) (layer "B.Cu") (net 20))
 (segment (start 37.02 50.51) (end 37.02 47.35) (width 0.25) (layer "B.Cu") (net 20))
 (segment (start 55.94 6.315) (end 55.94 12.36) (width 0.25) (layer "B.Cu") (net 20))
 (segment (start 115.6 8.1) (end 115.6 5.8) (width 0.25) (layer "B.Cu") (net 20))
 (segment (start 77.5 5.8) (end 77.5 5.34) (width 0.25) (layer "B.Cu") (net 20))
 (segment (start 116.81 50.625) (end 114.945 52.49) (width 0.25) (layer "B.Cu") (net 20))
 (segment (start 43.84 52.49) (end 43.66 52.49) (width 0.25) (layer "B.Cu") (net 20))
 (segment (start 43.66 52.49) (end 39 52.49) (width 0.25) (layer "B.Cu") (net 20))
 (segment (start 119.35 50.625) (end 116.81 50.625) (width 0.25) (layer "B.Cu") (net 20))
 (segment (start 54.02 14.28) (end 75.5 14.28) (width 0.25) (layer "B.Cu") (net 20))
 (segment (start 77.5 5.8) (end 77.5 12.28) (width 0.25) (layer "B.Cu") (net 20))
 (segment (start 200.9 49.88) (end 205.575 49.88) (width 0.25) (layer "B.Cu") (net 20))
 (segment (start 85.8 14.28) (end 109.42 14.28) (width 0.25) (layer "B.Cu") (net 20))
 (segment (start 39 52.49) (end 28.96 52.49) (width 0.25) (layer "B.Cu") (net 20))
 (segment (start 193.46 52.5) (end 196.08 49.88) (width 0.25) (layer "B.Cu") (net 20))
 (segment (start 28.5 52.49) (end 28.96 52.49) (width 0.25) (layer "B.Cu") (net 20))
 (segment (start 3.97 42.69) (end 6.51 42.69) (width 0.25) (layer "B.Cu") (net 20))
 (segment (start 114.945 52.49) (end 43.84 52.49) (width 0.25) (layer "B.Cu") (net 20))
 (segment (start 196.08 49.88) (end 200.9 49.88) (width 0.25) (layer "B.Cu") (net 20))
 (segment (start 210.195 49.865) (end 210.21 49.88) (width 0.25) (layer "B.Cu") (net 20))
 (segment (start 87.66 5.43) (end 87.66 5.8) (width 0.25) (layer "B.Cu") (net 20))
 (segment (start 205.555 49.89) (end 205.57 49.875) (width 0.25) (layer "B.Cu") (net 20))
 (segment (start 87.66 5.8) (end 87.66 12.42) (width 0.25) (layer "B.Cu") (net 20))
 (segment (start 55.95 2.655) (end 55.95 6.305) (width 0.25) (layer "B.Cu") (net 20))
 (segment (start 77.5 12.28) (end 75.5 14.28) (width 0.25) (layer "B.Cu") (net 20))
 (segment (start 37.02 50.51) (end 39 52.49) (width 0.25) (layer "B.Cu") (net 20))
 (segment (start 196.06 49.89) (end 196.05 49.89) (width 0.25) (layer "B.Cu") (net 20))
 (segment (start 55.94 12.36) (end 54.02 14.28) (width 0.25) (layer "B.Cu") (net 20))
 (segment (start 25 48.99) (end 10.77 48.99) (width 0.25) (layer "B.Cu") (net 20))
 (segment (start 55.95 6.305) (end 55.94 6.315) (width 0.25) (layer "B.Cu") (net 20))
 (segment (start 205.575 49.88) (end 205.59 49.865) (width 0.25) (layer "B.Cu") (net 20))
 (segment (start 75.5 14.28) (end 85.8 14.28) (width 0.25) (layer "B.Cu") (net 20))
 (segment (start 43.84 52.49) (end 41.74 50.39) (width 0.25) (layer "B.Cu") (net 20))
 (segment (start 41.74 50.39) (end 41.74 47.35) (width 0.25) (layer "B.Cu") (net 20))
 (segment (start 25 48.99) (end 28.5 52.49) (width 0.25) (layer "B.Cu") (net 20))
 (segment (start 109.42 14.28) (end 115.6 8.1) (width 0.25) (layer "B.Cu") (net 20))
 (segment (start 10.05 14.28) (end 54.02 14.28) (width 0.25) (layer "B.Cu") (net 20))
 (segment (start 3.97 42.69) (end 10.27 48.99) (width 0.25) (layer "B.Cu") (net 20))
 (segment (start 121.225 52.5) (end 193.46 52.5) (width 0.25) (layer "B.Cu") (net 20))
 (segment (start 9.05 42.69) (end 9.05 18.28) (width 0.25) (layer "B.Cu") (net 34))
 (segment (start 108.63 16.12) (end 117.83 6.92) (width 0.25) (layer "B.Cu") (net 34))
 (segment (start 117.83 6.92) (end 117.83 2.365) (width 0.25) (layer "B.Cu") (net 34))
 (segment (start 11.21 16.12) (end 108.63 16.12) (width 0.25) (layer "B.Cu") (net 34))
 (segment (start 9.05 18.28) (end 11.21 16.12) (width 0.25) (layer "B.Cu") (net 34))
 (segment (start 60.32 24.04) (end 64.41 19.95) (width 0.25) (layer "B.Cu") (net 15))
 (segment (start 64.41 19.95) (end 106.845 19.95) (width 0.25) (layer "B.Cu") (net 15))
 (segment (start 41.74 38.35) (end 56.05 24.04) (width 0.25) (layer "B.Cu") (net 15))
 (segment (start 56.05 24.04) (end 60.32 24.04) (width 0.25) (layer "B.Cu") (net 15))
 (segment (start 106.845 19.95) (end 124.43 2.365) (width 0.25) (layer "B.Cu") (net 15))
 (segment (start 172.86 14.35) (end 172.86 14.33) (width 0.25) (layer "F.Cu") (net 18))
 (segment (start 147.05 14.82) (end 134.595 2.365) (width 0.25) (layer "B.Cu") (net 18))
 (segment (start 207.84 19.78) (end 180.05 19.78) (width 0.25) (layer "B.Cu") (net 18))
 (segment (start 180.05 19.78) (end 175.09 14.82) (width 0.25) (layer "B.Cu") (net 18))
 (segment (start 172.82 14.82) (end 147.05 14.82) (width 0.25) (layer "B.Cu") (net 18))
 (segment (start 134.595 2.365) (end 134.59 2.365) (width 0.25) (layer "B.Cu") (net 18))
 (segment (start 210.21 22.15) (end 207.84 19.78) (width 0.25) (layer "B.Cu") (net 18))
 (segment (start 210.21 40.88) (end 210.21 22.15) (width 0.25) (layer "B.Cu") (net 18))
 (segment (start 175.09 14.82) (end 172.82 14.82) (width 0.25) (layer "B.Cu") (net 18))
 (segment (start 149.47 19.79) (end 132.05 2.37) (width 0.25) (layer "B.Cu") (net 9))
 (segment (start 205.59 40.865) (end 193.705 28.98) (width 0.25) (layer "B.Cu") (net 9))
 (segment (start 186.96 28.98) (end 177.77 19.79) (width 0.25) (layer "B.Cu") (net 9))
 (segment (start 132.05 2.37) (end 132.05 2.365) (width 0.25) (layer "B.Cu") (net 9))
 (segment (start 177.77 19.79) (end 149.47 19.79) (width 0.25) (layer "B.Cu") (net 9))
 (segment (start 193.705 28.98) (end 186.96 28.98) (width 0.25) (layer "B.Cu") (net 9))
 (segment (start 126.97 2.37) (end 126.97 2.365) (width 0.25) (layer "B.Cu") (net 3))
 (segment (start 172.82 43.11) (end 167.71 43.11) (width 0.25) (layer "B.Cu") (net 3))
 (segment (start 196.34 45.45) (end 175.18 45.45) (width 0.25) (layer "B.Cu") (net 3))
 (segment (start 200.9 40.89) (end 196.34 45.45) (width 0.25) (layer "B.Cu") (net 3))
 (segment (start 175.18 45.45) (end 172.84 43.11) (width 0.25) (layer "B.Cu") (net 3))
 (segment (start 167.71 43.11) (end 126.97 2.37) (width 0.25) (layer "B.Cu") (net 3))
 (segment (start 158.73 28.49) (end 158.72 28.49) (width 0.25) (layer "F.Cu") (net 12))
 (segment (start 158.68 28.98) (end 156.12 28.98) (width 0.25) (layer "B.Cu") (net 12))
 (segment (start 129.51 2.37) (end 129.51 2.365) (width 0.25) (layer "B.Cu") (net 12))
 (segment (start 156.12 28.98) (end 129.51 2.37) (width 0.25) (layer "B.Cu") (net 12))
 (segment (start 196.08 40.88) (end 189.13 33.93) (width 0.25) (layer "B.Cu") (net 12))
 (segment (start 163.63 33.93) (end 158.68 28.98) (width 0.25) (layer "B.Cu") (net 12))
 (segment (start 189.13 33.93) (end 163.63 33.93) (width 0.25) (layer "B.Cu") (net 12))
 (segment (start 113.06 6.12) (end 113.06 5.8) (width 0.25) (layer "B.Cu") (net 32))
 (segment (start 113.06 5.89) (end 113.06 5.8) (width 0.25) (layer "B.Cu") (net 32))
 (segment (start 108.18 11) (end 113.06 6.12) (width 0.25) (layer "B.Cu") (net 32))
 (segment (start 101.8 11) (end 108.18 11) (width 0.25) (layer "B.Cu") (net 32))
 (segment (start 86.86 8) (end 131.48 8) (width 0.25) (layer "F.Cu") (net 22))
 (segment (start 131.48 8) (end 137.115 2.365) (width 0.25) (layer "F.Cu") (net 22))
 (segment (start 85.12 5.8) (end 85.12 6.26) (width 0.25) (layer "F.Cu") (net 22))
 (segment (start 85.12 6.26) (end 86.86 8) (width 0.25) (layer "F.Cu") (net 22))
 (segment (start 137.115 2.365) (end 137.13 2.365) (width 0.25) (layer "F.Cu") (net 22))
 (segment (start 90.2 5.8) (end 90.2 4.3) (width 0.25) (layer "F.Cu") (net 23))
 (segment (start 90.8 3.7) (end 103.795 3.7) (width 0.25) (layer "F.Cu") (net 23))
 (segment (start 90.2 4.3) (end 90.8 3.7) (width 0.25) (layer "F.Cu") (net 23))
 (segment (start 103.795 3.7) (end 105.13 2.365) (width 0.25) (layer "F.Cu") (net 23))
 (segment (start 112.6 3.72) (end 113.935 3.72) (width 0.25) (layer "F.Cu") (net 31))
 (segment (start 113.935 3.72) (end 115.29 2.365) (width 0.25) (layer "F.Cu") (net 31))
 (segment (start 110.52 5.8) (end 112.6 3.72) (width 0.25) (layer "F.Cu") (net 31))
 (segment (start 111.395 3.72) (end 112.75 2.365) (width 0.25) (layer "F.Cu") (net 30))
 (segment (start 110.06 3.72) (end 111.395 3.72) (width 0.25) (layer "F.Cu") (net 30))
 (segment (start 107.98 5.8) (end 110.06 3.72) (width 0.25) (layer "F.Cu") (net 30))
 (segment (start 105.44 5.8) (end 107.52 3.72) (width 0.25) (layer "F.Cu") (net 29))
 (segment (start 107.52 3.72) (end 108.855 3.72) (width 0.25) (layer "F.Cu") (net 29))
 (segment (start 108.855 3.72) (end 110.21 2.365) (width 0.25) (layer "F.Cu") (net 29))
 (segment (start 106.325 3.71) (end 107.67 2.365) (width 0.25) (layer "F.Cu") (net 28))
 (segment (start 104.99 3.71) (end 106.325 3.71) (width 0.25) (layer "F.Cu") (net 28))
 (segment (start 102.9 5.8) (end 104.99 3.71) (width 0.25) (layer "F.Cu") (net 28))
 (segment (start 64.97 2.635) (end 64.95 2.655) (width 0.25) (layer "F.Cu") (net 21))
 (segment (start 79.435 2.655) (end 82.58 5.8) (width 0.25) (layer "F.Cu") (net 21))
 (segment (start 64.95 2.655) (end 64.95 6.305) (width 0.25) (layer "F.Cu") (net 21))
 (segment (start 64.95 2.655) (end 64.97 2.675) (width 0.25) (layer "F.Cu") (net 21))
 (segment (start 64.95 6.305) (end 64.94 6.315) (width 0.25) (layer "F.Cu") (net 21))
 (segment (start 64.95 2.655) (end 79.435 2.655) (width 0.25) (layer "F.Cu") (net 21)))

